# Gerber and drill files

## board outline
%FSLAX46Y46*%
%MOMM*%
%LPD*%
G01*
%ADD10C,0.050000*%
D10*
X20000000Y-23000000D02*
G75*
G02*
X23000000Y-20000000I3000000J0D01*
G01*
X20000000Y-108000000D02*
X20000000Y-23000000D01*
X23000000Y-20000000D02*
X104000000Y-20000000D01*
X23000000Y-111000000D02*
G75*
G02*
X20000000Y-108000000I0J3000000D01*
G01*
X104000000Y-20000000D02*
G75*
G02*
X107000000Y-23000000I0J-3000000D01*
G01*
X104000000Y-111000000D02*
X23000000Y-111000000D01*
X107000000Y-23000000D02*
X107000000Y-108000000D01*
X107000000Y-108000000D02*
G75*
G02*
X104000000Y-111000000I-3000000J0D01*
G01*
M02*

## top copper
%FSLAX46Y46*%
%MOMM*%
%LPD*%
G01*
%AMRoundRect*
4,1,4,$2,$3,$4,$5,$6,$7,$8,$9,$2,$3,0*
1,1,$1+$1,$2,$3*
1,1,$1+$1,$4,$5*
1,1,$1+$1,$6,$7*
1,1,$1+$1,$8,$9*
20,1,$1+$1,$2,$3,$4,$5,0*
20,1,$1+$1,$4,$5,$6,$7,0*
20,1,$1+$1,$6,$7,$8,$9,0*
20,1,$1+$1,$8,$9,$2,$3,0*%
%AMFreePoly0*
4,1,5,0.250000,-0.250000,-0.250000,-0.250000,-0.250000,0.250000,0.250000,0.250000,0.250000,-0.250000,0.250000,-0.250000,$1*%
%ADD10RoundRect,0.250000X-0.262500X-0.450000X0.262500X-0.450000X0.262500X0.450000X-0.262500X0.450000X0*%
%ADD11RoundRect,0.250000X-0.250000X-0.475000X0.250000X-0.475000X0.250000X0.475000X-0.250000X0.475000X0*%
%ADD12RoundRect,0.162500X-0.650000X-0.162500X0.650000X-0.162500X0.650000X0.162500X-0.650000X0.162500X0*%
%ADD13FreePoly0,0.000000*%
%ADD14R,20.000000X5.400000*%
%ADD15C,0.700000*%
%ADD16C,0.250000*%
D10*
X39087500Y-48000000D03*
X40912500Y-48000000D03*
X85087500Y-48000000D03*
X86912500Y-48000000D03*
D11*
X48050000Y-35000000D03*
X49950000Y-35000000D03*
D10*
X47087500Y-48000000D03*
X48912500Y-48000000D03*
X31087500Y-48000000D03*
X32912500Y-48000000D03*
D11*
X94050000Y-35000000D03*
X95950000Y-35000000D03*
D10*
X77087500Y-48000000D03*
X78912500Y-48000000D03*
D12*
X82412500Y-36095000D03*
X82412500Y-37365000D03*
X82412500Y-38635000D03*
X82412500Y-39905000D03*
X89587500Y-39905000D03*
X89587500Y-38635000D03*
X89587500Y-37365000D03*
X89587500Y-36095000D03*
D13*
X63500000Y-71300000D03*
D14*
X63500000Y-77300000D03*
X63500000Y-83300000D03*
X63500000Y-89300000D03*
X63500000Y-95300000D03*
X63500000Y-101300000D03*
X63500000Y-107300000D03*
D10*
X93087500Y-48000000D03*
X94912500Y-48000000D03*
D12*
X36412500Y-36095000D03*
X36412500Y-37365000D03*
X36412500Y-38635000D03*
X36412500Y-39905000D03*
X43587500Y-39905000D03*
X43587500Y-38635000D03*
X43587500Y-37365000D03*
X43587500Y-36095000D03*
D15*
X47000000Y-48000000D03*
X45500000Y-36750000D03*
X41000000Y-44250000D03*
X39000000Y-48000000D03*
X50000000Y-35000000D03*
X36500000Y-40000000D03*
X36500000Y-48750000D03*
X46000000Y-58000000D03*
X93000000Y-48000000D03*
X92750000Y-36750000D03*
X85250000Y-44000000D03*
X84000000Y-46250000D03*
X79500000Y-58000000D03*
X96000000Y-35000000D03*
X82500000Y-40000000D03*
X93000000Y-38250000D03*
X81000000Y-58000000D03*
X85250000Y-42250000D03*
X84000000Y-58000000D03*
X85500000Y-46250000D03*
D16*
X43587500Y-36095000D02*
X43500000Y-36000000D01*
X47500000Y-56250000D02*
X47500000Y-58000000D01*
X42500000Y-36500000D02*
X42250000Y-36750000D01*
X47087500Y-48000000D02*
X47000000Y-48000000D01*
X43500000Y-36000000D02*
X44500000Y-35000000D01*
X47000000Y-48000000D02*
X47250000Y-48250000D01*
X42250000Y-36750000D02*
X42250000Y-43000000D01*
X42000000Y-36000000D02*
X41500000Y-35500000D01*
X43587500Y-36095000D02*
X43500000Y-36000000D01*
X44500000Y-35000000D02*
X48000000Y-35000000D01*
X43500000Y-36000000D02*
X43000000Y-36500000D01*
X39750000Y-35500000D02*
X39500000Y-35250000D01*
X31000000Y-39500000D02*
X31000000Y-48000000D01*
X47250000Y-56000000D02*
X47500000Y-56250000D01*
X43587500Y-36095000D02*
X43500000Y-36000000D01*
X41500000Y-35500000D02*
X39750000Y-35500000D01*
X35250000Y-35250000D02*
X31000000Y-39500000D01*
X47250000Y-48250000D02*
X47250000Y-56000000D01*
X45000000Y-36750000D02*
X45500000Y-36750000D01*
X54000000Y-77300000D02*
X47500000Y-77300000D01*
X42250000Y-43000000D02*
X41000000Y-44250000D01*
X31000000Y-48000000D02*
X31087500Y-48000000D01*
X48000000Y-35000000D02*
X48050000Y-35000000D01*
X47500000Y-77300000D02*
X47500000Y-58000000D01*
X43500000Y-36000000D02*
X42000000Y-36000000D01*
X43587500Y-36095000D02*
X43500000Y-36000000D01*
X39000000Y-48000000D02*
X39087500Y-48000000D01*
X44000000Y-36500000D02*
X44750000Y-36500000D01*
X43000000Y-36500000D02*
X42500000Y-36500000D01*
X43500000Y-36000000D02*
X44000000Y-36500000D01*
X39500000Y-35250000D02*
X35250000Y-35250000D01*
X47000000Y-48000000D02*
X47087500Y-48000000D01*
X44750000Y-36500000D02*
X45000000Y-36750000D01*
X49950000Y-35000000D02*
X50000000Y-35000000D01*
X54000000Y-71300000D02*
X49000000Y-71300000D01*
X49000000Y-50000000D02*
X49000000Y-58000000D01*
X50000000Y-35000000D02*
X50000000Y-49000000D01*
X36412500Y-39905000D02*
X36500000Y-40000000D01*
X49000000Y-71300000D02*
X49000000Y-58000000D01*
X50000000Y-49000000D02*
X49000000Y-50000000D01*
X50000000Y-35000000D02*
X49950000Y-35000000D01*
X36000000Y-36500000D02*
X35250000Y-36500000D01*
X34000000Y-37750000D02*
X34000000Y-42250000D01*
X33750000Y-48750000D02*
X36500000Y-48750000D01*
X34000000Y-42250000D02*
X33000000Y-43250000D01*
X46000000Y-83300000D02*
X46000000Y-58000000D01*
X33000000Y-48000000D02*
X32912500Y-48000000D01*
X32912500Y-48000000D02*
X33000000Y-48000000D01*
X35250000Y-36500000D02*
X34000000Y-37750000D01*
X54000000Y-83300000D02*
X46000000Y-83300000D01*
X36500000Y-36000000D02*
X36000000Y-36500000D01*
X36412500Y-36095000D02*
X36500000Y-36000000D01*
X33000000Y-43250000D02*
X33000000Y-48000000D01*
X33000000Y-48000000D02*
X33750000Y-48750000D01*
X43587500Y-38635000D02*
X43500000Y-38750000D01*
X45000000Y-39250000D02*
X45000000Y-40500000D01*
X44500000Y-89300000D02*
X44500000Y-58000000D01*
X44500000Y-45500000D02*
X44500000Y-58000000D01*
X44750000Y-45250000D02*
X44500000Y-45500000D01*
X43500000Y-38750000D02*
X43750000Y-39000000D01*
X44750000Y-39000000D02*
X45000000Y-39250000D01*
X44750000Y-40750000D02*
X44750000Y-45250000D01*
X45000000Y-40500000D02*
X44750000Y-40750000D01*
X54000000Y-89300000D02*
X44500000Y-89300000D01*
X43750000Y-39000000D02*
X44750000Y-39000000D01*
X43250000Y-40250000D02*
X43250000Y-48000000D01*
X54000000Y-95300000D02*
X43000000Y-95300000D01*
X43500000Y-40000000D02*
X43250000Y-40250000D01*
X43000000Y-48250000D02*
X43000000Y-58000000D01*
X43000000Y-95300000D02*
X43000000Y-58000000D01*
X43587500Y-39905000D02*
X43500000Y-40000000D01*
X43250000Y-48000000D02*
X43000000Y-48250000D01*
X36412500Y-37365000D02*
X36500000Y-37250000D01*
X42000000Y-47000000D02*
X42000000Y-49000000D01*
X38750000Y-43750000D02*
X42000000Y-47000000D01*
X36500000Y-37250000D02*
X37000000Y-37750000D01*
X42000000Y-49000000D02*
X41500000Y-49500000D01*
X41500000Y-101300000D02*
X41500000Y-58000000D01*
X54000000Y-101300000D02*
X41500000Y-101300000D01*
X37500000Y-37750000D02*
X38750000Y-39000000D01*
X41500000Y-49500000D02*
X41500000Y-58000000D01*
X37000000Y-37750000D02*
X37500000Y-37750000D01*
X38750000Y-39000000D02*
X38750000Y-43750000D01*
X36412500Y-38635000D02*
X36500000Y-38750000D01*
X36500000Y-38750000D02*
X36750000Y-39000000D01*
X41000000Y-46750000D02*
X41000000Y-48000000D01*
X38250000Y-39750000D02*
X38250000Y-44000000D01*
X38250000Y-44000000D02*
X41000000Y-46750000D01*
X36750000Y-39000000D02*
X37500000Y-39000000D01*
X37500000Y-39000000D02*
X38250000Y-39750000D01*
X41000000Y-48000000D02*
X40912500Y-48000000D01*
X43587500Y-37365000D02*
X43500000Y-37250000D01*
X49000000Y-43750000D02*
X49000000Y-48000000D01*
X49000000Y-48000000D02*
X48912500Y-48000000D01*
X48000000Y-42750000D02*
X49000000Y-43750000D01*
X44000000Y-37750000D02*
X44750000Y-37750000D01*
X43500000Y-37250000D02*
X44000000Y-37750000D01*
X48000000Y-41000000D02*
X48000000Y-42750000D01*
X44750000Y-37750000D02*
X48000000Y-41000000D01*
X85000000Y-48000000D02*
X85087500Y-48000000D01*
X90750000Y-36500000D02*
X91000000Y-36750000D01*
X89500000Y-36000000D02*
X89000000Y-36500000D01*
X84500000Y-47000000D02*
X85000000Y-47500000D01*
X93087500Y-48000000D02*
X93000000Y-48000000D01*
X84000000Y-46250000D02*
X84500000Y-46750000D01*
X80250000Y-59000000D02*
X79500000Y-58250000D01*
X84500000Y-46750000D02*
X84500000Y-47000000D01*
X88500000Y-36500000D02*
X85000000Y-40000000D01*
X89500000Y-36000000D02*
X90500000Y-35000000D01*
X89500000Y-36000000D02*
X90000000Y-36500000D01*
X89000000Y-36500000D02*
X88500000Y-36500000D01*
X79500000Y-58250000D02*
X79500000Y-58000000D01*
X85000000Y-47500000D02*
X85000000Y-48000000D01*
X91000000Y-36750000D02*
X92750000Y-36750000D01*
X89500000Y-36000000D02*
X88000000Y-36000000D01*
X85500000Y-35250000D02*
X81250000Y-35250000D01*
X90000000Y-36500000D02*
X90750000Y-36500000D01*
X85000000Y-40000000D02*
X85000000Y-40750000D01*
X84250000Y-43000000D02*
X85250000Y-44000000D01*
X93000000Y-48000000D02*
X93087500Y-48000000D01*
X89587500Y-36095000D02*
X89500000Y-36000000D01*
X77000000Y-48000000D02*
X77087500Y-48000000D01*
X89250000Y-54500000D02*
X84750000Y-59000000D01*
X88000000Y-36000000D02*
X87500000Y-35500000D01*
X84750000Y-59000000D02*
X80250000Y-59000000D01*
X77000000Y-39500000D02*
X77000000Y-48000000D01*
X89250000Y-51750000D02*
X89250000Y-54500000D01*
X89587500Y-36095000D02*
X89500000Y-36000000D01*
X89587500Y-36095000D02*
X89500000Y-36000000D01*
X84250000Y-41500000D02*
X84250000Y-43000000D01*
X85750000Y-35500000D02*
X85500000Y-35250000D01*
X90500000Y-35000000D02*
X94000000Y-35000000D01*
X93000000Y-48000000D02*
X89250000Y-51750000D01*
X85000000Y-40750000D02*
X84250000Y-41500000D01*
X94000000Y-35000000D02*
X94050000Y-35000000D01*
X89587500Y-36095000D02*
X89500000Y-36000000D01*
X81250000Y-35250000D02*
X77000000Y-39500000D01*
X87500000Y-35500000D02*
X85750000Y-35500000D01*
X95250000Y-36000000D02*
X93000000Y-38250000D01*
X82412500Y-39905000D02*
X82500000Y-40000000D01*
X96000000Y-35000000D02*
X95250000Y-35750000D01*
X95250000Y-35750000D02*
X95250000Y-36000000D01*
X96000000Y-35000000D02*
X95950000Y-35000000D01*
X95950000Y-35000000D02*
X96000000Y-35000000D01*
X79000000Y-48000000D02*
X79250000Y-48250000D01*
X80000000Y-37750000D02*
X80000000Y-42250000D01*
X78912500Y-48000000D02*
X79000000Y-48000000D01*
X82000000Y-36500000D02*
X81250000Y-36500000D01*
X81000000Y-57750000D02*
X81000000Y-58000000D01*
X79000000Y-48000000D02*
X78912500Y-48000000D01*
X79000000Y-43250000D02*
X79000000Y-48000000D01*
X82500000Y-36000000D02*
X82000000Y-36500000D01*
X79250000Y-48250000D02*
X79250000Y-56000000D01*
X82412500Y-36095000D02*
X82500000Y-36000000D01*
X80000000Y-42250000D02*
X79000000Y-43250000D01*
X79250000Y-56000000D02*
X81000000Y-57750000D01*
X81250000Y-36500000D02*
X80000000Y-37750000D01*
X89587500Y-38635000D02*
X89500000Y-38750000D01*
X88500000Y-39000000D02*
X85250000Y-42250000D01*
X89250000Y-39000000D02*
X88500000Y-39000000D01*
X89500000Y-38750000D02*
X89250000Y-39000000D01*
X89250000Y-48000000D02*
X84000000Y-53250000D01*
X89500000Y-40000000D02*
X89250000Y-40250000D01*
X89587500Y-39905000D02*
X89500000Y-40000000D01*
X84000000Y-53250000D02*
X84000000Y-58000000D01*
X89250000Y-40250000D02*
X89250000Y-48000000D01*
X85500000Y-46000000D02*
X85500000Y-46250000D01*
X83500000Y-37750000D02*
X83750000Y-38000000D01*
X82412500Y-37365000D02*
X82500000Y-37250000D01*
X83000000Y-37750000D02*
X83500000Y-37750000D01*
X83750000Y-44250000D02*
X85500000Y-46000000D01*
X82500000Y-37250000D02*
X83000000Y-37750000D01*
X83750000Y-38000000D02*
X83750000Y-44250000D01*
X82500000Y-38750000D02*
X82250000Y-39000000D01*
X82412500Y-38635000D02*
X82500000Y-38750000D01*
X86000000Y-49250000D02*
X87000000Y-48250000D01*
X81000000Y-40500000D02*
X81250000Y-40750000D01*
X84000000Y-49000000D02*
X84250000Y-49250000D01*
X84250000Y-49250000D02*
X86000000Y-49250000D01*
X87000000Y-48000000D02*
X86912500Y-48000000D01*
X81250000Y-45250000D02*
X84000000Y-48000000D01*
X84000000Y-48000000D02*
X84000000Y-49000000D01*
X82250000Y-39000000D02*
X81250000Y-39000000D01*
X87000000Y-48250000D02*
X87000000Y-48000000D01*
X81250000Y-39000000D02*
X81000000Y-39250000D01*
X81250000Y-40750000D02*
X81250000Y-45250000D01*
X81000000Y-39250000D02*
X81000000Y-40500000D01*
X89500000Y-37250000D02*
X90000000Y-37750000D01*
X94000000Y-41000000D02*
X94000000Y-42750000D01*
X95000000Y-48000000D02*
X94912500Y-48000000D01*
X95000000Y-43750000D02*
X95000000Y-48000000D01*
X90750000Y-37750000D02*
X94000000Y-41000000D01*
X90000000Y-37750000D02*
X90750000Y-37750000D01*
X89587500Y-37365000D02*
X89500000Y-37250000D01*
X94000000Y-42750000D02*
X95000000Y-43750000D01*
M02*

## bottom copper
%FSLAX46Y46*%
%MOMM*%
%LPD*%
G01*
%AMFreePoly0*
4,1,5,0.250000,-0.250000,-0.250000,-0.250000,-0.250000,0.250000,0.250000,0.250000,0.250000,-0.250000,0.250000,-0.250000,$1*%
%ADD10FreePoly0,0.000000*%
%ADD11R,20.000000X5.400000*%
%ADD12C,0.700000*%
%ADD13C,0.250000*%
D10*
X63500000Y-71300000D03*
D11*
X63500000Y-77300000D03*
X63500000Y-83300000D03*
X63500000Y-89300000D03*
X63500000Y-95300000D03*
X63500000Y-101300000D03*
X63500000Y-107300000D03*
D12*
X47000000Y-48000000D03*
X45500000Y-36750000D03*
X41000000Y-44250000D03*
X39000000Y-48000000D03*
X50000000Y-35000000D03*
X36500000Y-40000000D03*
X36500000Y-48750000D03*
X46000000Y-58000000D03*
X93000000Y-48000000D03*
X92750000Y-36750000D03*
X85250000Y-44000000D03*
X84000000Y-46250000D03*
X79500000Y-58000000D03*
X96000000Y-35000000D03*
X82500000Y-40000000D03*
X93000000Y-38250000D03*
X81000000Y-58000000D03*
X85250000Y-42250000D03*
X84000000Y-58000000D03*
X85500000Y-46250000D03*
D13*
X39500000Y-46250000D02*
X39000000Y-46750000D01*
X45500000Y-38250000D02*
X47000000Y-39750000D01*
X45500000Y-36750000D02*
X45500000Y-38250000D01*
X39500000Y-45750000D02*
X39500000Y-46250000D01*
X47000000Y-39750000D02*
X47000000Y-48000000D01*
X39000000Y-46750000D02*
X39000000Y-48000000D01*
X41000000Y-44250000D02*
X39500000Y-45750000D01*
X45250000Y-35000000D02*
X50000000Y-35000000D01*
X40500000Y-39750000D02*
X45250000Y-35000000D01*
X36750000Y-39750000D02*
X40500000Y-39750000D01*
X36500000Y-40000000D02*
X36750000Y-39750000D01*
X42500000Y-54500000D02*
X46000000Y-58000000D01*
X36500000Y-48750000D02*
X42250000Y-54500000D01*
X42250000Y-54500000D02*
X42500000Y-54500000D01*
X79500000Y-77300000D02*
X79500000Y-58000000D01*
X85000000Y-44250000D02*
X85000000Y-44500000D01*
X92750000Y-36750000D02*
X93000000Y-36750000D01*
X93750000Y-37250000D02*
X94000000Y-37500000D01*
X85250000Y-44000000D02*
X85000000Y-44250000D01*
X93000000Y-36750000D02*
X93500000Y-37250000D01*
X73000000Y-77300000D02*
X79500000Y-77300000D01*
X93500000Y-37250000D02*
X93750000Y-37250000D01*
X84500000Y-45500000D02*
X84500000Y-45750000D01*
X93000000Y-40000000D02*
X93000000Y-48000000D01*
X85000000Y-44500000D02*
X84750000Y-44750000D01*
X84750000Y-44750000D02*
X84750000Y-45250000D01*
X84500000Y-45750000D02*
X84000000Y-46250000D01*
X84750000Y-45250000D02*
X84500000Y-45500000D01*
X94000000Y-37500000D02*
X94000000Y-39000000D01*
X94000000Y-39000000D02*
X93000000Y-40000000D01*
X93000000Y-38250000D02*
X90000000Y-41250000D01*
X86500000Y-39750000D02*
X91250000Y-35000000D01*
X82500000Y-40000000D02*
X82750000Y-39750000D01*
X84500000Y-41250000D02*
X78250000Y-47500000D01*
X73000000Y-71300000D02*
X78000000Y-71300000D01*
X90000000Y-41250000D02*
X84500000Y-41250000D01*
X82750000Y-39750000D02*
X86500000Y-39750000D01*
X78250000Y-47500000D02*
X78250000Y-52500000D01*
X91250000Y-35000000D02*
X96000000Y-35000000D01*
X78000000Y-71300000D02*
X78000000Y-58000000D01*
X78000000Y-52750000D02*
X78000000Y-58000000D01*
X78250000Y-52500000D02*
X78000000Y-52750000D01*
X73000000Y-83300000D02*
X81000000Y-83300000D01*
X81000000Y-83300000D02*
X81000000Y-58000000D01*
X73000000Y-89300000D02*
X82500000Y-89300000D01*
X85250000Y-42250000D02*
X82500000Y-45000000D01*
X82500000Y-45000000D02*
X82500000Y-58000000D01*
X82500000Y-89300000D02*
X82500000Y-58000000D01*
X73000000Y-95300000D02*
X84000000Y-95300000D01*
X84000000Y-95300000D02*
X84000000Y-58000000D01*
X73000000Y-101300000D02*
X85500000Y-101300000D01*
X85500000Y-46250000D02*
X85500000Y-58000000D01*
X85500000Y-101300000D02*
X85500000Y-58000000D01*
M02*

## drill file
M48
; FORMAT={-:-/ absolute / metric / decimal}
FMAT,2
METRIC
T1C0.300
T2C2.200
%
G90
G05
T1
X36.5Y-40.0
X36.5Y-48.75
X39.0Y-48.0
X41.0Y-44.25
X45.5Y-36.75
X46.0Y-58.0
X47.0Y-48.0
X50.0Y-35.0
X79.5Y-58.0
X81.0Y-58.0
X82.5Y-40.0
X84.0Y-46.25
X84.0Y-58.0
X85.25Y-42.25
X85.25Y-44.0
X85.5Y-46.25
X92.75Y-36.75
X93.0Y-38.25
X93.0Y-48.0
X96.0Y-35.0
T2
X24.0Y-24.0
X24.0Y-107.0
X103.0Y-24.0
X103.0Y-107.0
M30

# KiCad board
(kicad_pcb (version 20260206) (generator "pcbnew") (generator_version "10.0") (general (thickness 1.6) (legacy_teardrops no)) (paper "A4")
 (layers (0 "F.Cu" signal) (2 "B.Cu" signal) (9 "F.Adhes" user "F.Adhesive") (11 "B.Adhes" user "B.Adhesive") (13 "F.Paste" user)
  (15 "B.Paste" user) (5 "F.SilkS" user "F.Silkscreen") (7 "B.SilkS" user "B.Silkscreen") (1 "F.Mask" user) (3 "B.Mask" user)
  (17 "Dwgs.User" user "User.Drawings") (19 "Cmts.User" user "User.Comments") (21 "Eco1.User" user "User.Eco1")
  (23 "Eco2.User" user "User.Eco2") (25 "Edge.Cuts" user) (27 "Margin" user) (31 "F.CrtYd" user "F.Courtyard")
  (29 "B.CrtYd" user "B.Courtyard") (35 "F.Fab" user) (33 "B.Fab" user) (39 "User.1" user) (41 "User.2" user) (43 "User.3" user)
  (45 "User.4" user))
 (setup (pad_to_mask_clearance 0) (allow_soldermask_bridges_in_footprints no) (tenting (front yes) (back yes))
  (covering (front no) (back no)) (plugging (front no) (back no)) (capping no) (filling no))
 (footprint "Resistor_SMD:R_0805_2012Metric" (layer "F.Cu") (at 40 48)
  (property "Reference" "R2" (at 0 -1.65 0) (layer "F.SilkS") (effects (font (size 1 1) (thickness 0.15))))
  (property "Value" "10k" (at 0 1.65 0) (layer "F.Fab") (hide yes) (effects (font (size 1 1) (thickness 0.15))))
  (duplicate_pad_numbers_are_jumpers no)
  (pad "1" smd roundrect (at -0.9125 0) (size 1.025 1.4) (layers "F.Cu" "F.Mask" "F.Paste") (roundrect_rratio 0.243902) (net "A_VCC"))
  (pad "2" smd roundrect (at 0.9125 0) (size 1.025 1.4) (layers "F.Cu" "F.Mask" "F.Paste") (roundrect_rratio 0.243902) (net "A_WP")))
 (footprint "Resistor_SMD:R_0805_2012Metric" (layer "F.Cu") (at 86 48)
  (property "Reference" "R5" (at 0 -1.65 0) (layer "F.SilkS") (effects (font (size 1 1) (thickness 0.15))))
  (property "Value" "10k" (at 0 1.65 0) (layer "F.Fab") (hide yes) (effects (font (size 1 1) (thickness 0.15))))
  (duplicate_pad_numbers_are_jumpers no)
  (pad "1" smd roundrect (at -0.9125 0) (size 1.025 1.4) (layers "F.Cu" "F.Mask" "F.Paste") (roundrect_rratio 0.243902) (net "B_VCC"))
  (pad "2" smd roundrect (at 0.9125 0) (size 1.025 1.4) (layers "F.Cu" "F.Mask" "F.Paste") (roundrect_rratio 0.243902) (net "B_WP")))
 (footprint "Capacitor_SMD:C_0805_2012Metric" (layer "F.Cu") (at 49 35)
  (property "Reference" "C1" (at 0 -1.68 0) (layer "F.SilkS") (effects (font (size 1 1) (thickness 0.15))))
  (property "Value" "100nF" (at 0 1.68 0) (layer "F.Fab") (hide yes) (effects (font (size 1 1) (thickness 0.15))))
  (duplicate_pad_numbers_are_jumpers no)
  (pad "1" smd roundrect (at -0.95 0) (size 1 1.45) (layers "F.Cu" "F.Mask" "F.Paste") (roundrect_rratio 0.25) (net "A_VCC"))
  (pad "2" smd roundrect (at 0.95 0) (size 1 1.45) (layers "F.Cu" "F.Mask" "F.Paste") (roundrect_rratio 0.25) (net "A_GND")))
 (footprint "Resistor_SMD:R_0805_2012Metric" (layer "F.Cu") (at 48 48)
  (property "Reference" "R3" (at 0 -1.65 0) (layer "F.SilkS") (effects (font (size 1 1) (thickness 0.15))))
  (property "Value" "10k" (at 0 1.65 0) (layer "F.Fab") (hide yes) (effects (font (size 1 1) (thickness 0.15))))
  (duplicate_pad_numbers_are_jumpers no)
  (pad "1" smd roundrect (at -0.9125 0) (size 1.025 1.4) (layers "F.Cu" "F.Mask" "F.Paste") (roundrect_rratio 0.243902) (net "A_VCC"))
  (pad "2" smd roundrect (at 0.9125 0) (size 1.025 1.4) (layers "F.Cu" "F.Mask" "F.Paste") (roundrect_rratio 0.243902) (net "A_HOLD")))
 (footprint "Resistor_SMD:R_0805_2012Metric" (layer "F.Cu") (at 32 48)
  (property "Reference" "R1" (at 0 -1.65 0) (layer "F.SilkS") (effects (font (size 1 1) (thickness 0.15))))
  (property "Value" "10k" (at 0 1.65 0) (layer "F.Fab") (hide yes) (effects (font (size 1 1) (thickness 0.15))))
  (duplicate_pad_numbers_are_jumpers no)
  (pad "1" smd roundrect (at -0.9125 0) (size 1.025 1.4) (layers "F.Cu" "F.Mask" "F.Paste") (roundrect_rratio 0.243902) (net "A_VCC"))
  (pad "2" smd roundrect (at 0.9125 0) (size 1.025 1.4) (layers "F.Cu" "F.Mask" "F.Paste") (roundrect_rratio 0.243902) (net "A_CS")))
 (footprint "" (layer "F.Cu") (at 103 107)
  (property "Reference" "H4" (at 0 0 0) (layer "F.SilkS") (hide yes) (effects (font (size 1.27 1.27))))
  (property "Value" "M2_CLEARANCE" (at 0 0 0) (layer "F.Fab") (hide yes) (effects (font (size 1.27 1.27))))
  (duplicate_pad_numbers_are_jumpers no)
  (pad "" np_thru_hole circle (at 0 0) (size 2.2 2.2) (drill 2.2) (layers "*.Cu")))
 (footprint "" (layer "F.Cu") (at 24 24)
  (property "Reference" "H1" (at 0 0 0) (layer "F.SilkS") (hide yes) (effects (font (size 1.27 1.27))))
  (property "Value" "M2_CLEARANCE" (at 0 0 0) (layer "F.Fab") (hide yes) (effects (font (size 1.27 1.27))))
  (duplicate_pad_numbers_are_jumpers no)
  (pad "" np_thru_hole circle (at 0 0) (size 2.2 2.2) (drill 2.2) (layers "*.Cu")))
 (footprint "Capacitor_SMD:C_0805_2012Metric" (layer "F.Cu") (at 95 35)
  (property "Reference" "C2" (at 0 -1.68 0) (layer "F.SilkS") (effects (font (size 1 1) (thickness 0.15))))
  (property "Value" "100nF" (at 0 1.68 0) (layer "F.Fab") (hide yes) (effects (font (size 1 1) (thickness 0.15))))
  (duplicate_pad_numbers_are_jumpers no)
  (pad "1" smd roundrect (at -0.95 0) (size 1 1.45) (layers "F.Cu" "F.Mask" "F.Paste") (roundrect_rratio 0.25) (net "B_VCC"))
  (pad "2" smd roundrect (at 0.95 0) (size 1 1.45) (layers "F.Cu" "F.Mask" "F.Paste") (roundrect_rratio 0.25) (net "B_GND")))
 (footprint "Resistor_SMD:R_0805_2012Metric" (layer "F.Cu") (at 78 48)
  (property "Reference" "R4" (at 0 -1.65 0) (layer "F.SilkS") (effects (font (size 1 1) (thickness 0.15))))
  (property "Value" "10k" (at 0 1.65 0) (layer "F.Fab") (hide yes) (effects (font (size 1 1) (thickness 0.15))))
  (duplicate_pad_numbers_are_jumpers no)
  (pad "1" smd roundrect (at -0.9125 0) (size 1.025 1.4) (layers "F.Cu" "F.Mask" "F.Paste") (roundrect_rratio 0.243902) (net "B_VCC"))
  (pad "2" smd roundrect (at 0.9125 0) (size 1.025 1.4) (layers "F.Cu" "F.Mask" "F.Paste") (roundrect_rratio 0.243902) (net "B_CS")))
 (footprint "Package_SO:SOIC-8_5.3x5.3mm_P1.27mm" (layer "F.Cu") (at 86 38)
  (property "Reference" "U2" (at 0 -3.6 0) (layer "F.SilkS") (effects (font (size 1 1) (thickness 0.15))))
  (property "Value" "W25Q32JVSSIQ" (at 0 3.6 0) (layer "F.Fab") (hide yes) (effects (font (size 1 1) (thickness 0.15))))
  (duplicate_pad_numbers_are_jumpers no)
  (pad "1" smd roundrect (at -3.5875 -1.905) (size 1.625 0.65) (layers "F.Cu" "F.Mask" "F.Paste") (roundrect_rratio 0.25) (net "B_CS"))
  (pad "2" smd roundrect (at -3.5875 -0.635) (size 1.625 0.65) (layers "F.Cu" "F.Mask" "F.Paste") (roundrect_rratio 0.25) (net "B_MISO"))
  (pad "3" smd roundrect (at -3.5875 0.635) (size 1.625 0.65) (layers "F.Cu" "F.Mask" "F.Paste") (roundrect_rratio 0.25) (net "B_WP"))
  (pad "4" smd roundrect (at -3.5875 1.905) (size 1.625 0.65) (layers "F.Cu" "F.Mask" "F.Paste") (roundrect_rratio 0.25) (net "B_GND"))
  (pad "5" smd roundrect (at 3.5875 1.905) (size 1.625 0.65) (layers "F.Cu" "F.Mask" "F.Paste") (roundrect_rratio 0.25) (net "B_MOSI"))
  (pad "6" smd roundrect (at 3.5875 0.635) (size 1.625 0.65) (layers "F.Cu" "F.Mask" "F.Paste") (roundrect_rratio 0.25) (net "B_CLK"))
  (pad "7" smd roundrect (at 3.5875 -0.635) (size 1.625 0.65) (layers "F.Cu" "F.Mask" "F.Paste") (roundrect_rratio 0.25) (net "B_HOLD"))
  (pad "8" smd roundrect (at 3.5875 -1.905) (size 1.625 0.65) (layers "F.Cu" "F.Mask" "F.Paste") (roundrect_rratio 0.25) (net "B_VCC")))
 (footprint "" (layer "F.Cu") (at 103 24)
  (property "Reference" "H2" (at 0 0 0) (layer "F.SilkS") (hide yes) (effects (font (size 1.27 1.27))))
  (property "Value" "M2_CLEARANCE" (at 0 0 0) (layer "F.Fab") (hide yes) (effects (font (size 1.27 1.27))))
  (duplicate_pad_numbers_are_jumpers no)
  (pad "" np_thru_hole circle (at 0 0) (size 2.2 2.2) (drill 2.2) (layers "*.Cu")))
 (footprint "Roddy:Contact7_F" (layer "F.Cu") (at 63.5 0)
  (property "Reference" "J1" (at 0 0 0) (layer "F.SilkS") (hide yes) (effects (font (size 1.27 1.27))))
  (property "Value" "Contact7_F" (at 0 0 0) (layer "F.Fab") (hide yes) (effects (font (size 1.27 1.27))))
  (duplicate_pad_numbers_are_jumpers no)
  (pad "1" smd custom (at 0 71.3) (size 0.5 0.5) (layers "F.Cu" "F.Mask") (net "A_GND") (solder_mask_margin 0.05) (thermal_bridge_angle 45)
   (options (clearance outline) (anchor rect)) (primitives))
  (pad "2" smd rect (at 0 77.3) (size 20 5.4) (layers "F.Cu" "F.Mask") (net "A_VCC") (solder_mask_margin 0.05) (thermal_bridge_angle 45))
  (pad "3" smd rect (at 0 83.3) (size 20 5.4) (layers "F.Cu" "F.Mask") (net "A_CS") (solder_mask_margin 0.05) (thermal_bridge_angle 45))
  (pad "4" smd rect (at 0 89.3) (size 20 5.4) (layers "F.Cu" "F.Mask") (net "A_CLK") (solder_mask_margin 0.05) (thermal_bridge_angle 45))
  (pad "5" smd rect (at 0 95.3) (size 20 5.4) (layers "F.Cu" "F.Mask") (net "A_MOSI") (solder_mask_margin 0.05) (thermal_bridge_angle 45))
  (pad "6" smd rect (at 0 101.3) (size 20 5.4) (layers "F.Cu" "F.Mask") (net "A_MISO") (solder_mask_margin 0.05) (thermal_bridge_angle 45))
  (pad "7" smd rect (at 0 107.3) (size 20 5.4) (layers "F.Cu" "F.Mask") (solder_mask_margin 0.05) (thermal_bridge_angle 45)))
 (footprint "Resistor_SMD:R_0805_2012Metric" (layer "F.Cu") (at 94 48)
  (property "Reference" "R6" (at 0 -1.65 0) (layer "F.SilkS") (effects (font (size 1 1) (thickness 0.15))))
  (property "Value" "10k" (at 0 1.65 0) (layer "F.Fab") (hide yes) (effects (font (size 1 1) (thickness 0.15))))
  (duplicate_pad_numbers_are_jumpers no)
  (pad "1" smd roundrect (at -0.9125 0) (size 1.025 1.4) (layers "F.Cu" "F.Mask" "F.Paste") (roundrect_rratio 0.243902) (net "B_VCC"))
  (pad "2" smd roundrect (at 0.9125 0) (size 1.025 1.4) (layers "F.Cu" "F.Mask" "F.Paste") (roundrect_rratio 0.243902) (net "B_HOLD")))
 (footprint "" (layer "F.Cu") (at 24 107)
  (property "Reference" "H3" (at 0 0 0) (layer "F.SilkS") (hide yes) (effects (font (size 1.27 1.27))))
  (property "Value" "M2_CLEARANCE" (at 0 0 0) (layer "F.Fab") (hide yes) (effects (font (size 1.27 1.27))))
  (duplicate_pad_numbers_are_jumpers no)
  (pad "" np_thru_hole circle (at 0 0) (size 2.2 2.2) (drill 2.2) (layers "*.Cu")))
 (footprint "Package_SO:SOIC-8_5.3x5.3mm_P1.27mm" (layer "F.Cu") (at 40 38)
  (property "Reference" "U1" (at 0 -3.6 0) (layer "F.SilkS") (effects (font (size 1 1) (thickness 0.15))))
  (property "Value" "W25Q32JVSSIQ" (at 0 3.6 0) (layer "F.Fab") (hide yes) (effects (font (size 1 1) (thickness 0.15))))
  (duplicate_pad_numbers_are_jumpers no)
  (pad "1" smd roundrect (at -3.5875 -1.905) (size 1.625 0.65) (layers "F.Cu" "F.Mask" "F.Paste") (roundrect_rratio 0.25) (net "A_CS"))
  (pad "2" smd roundrect (at -3.5875 -0.635) (size 1.625 0.65) (layers "F.Cu" "F.Mask" "F.Paste") (roundrect_rratio 0.25) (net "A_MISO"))
  (pad "3" smd roundrect (at -3.5875 0.635) (size 1.625 0.65) (layers "F.Cu" "F.Mask" "F.Paste") (roundrect_rratio 0.25) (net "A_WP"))
  (pad "4" smd roundrect (at -3.5875 1.905) (size 1.625 0.65) (layers "F.Cu" "F.Mask" "F.Paste") (roundrect_rratio 0.25) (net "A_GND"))
  (pad "5" smd roundrect (at 3.5875 1.905) (size 1.625 0.65) (layers "F.Cu" "F.Mask" "F.Paste") (roundrect_rratio 0.25) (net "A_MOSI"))
  (pad "6" smd roundrect (at 3.5875 0.635) (size 1.625 0.65) (layers "F.Cu" "F.Mask" "F.Paste") (roundrect_rratio 0.25) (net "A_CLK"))
  (pad "7" smd roundrect (at 3.5875 -0.635) (size 1.625 0.65) (layers "F.Cu" "F.Mask" "F.Paste") (roundrect_rratio 0.25) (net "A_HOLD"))
  (pad "8" smd roundrect (at 3.5875 -1.905) (size 1.625 0.65) (layers "F.Cu" "F.Mask" "F.Paste") (roundrect_rratio 0.25) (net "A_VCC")))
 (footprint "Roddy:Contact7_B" (layer "B.Cu") (at 63.5 0)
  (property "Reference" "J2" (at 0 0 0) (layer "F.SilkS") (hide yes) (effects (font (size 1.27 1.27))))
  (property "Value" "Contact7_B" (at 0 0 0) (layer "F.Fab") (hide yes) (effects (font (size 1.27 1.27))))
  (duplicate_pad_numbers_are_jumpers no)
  (pad "1" smd custom (at 0 71.3) (size 0.5 0.5) (layers "B.Cu" "B.Mask") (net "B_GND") (solder_mask_margin 0.05) (thermal_bridge_angle 45)
   (options (clearance outline) (anchor rect)) (primitives))
  (pad "2" smd rect (at 0 77.3) (size 20 5.4) (layers "B.Cu" "B.Mask") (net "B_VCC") (solder_mask_margin 0.05) (thermal_bridge_angle 45))
  (pad "3" smd rect (at 0 83.3) (size 20 5.4) (layers "B.Cu" "B.Mask") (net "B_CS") (solder_mask_margin 0.05) (thermal_bridge_angle 45))
  (pad "4" smd rect (at 0 89.3) (size 20 5.4) (layers "B.Cu" "B.Mask") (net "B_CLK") (solder_mask_margin 0.05) (thermal_bridge_angle 45))
  (pad "5" smd rect (at 0 95.3) (size 20 5.4) (layers "B.Cu" "B.Mask") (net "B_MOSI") (solder_mask_margin 0.05) (thermal_bridge_angle 45))
  (pad "6" smd rect (at 0 101.3) (size 20 5.4) (layers "B.Cu" "B.Mask") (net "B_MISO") (solder_mask_margin 0.05) (thermal_bridge_angle 45))
  (pad "7" smd rect (at 0 107.3) (size 20 5.4) (layers "B.Cu" "B.Mask") (solder_mask_margin 0.05) (thermal_bridge_angle 45)))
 (gr_arc (start 20 23) (mid 20.878679 20.878679) (end 23 20) (stroke (width 0.05) (type default)) (layer "Edge.Cuts"))
 (gr_line (start 20 108) (end 20 23) (stroke (width 0.05) (type default)) (layer "Edge.Cuts"))
 (gr_line (start 23 20) (end 104 20) (stroke (width 0.05) (type default)) (layer "Edge.Cuts"))
 (gr_arc (start 23 111) (mid 20.878679 110.12132) (end 20 108) (stroke (width 0.05) (type default)) (layer "Edge.Cuts"))
 (gr_arc (start 104 20) (mid 106.12132 20.878679) (end 107 23) (stroke (width 0.05) (type default)) (layer "Edge.Cuts"))
 (gr_line (start 104 111) (end 23 111) (stroke (width 0.05) (type default)) (layer "Edge.Cuts"))
 (gr_line (start 107 23) (end 107 108) (stroke (width 0.05) (type default)) (layer "Edge.Cuts"))
 (gr_arc (start 107 108) (mid 106.12132 110.12132) (end 104 111) (stroke (width 0.05) (type default)) (layer "Edge.Cuts"))
 (segment (start 43.5875 36.095) (end 43.5 36) (width 0.25) (layer "F.Cu") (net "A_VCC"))
 (segment (start 47.5 56.25) (end 47.5 58) (width 0.25) (layer "F.Cu") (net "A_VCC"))
 (segment (start 42.5 36.5) (end 42.25 36.75) (width 0.25) (layer "F.Cu") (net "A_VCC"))
 (segment (start 47.0875 48) (end 47 48) (width 0.25) (layer "F.Cu") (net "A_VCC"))
 (segment (start 43.5 36) (end 44.5 35) (width 0.25) (layer "F.Cu") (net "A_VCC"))
 (segment (start 47 48) (end 47.25 48.25) (width 0.25) (layer "F.Cu") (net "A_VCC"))
 (segment (start 42.25 36.75) (end 42.25 43) (width 0.25) (layer "F.Cu") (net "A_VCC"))
 (segment (start 42 36) (end 41.5 35.5) (width 0.25) (layer "F.Cu") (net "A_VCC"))
 (segment (start 43.5875 36.095) (end 43.5 36) (width 0.25) (layer "F.Cu") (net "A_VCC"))
 (segment (start 44.5 35) (end 48 35) (width 0.25) (layer "F.Cu") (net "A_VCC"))
 (segment (start 43.5 36) (end 43 36.5) (width 0.25) (layer "F.Cu") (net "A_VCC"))
 (segment (start 39.75 35.5) (end 39.5 35.25) (width 0.25) (layer "F.Cu") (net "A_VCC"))
 (segment (start 31 39.5) (end 31 48) (width 0.25) (layer "F.Cu") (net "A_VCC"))
 (segment (start 47.25 56) (end 47.5 56.25) (width 0.25) (layer "F.Cu") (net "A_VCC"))
 (segment (start 43.5875 36.095) (end 43.5 36) (width 0.25) (layer "F.Cu") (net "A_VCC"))
 (segment (start 41.5 35.5) (end 39.75 35.5) (width 0.25) (layer "F.Cu") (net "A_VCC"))
 (segment (start 35.25 35.25) (end 31 39.5) (width 0.25) (layer "F.Cu") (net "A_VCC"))
 (segment (start 47.25 48.25) (end 47.25 56) (width 0.25) (layer "F.Cu") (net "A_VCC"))
 (segment (start 45 36.75) (end 45.5 36.75) (width 0.25) (layer "F.Cu") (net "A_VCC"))
 (segment (start 54 77.3) (end 47.5 77.3) (width 0.25) (layer "F.Cu") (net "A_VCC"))
 (segment (start 42.25 43) (end 41 44.25) (width 0.25) (layer "F.Cu") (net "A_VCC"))
 (segment (start 31 48) (end 31.0875 48) (width 0.25) (layer "F.Cu") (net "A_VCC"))
 (segment (start 48 35) (end 48.05 35) (width 0.25) (layer "F.Cu") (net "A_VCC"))
 (segment (start 47.5 77.3) (end 47.5 58) (width 0.25) (layer "F.Cu") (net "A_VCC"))
 (segment (start 43.5 36) (end 42 36) (width 0.25) (layer "F.Cu") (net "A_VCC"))
 (segment (start 43.5875 36.095) (end 43.5 36) (width 0.25) (layer "F.Cu") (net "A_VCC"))
 (segment (start 39 48) (end 39.0875 48) (width 0.25) (layer "F.Cu") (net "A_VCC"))
 (segment (start 44 36.5) (end 44.75 36.5) (width 0.25) (layer "F.Cu") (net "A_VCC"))
 (segment (start 43 36.5) (end 42.5 36.5) (width 0.25) (layer "F.Cu") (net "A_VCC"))
 (segment (start 43.5 36) (end 44 36.5) (width 0.25) (layer "F.Cu") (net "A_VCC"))
 (segment (start 39.5 35.25) (end 35.25 35.25) (width 0.25) (layer "F.Cu") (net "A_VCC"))
 (segment (start 47 48) (end 47.0875 48) (width 0.25) (layer "F.Cu") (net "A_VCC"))
 (segment (start 44.75 36.5) (end 45 36.75) (width 0.25) (layer "F.Cu") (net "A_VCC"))
 (via (at 47 48) (size 0.7) (drill 0.3) (layers "F.Cu" "B.Cu") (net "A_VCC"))
 (via (at 45.5 36.75) (size 0.7) (drill 0.3) (layers "F.Cu" "B.Cu") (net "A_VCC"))
 (via (at 41 44.25) (size 0.7) (drill 0.3) (layers "F.Cu" "B.Cu") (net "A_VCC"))
 (via (at 39 48) (size 0.7) (drill 0.3) (layers "F.Cu" "B.Cu") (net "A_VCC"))
 (segment (start 39.5 46.25) (end 39 46.75) (width 0.25) (layer "B.Cu") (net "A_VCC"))
 (segment (start 45.5 38.25) (end 47 39.75) (width 0.25) (layer "B.Cu") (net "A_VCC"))
 (segment (start 45.5 36.75) (end 45.5 38.25) (width 0.25) (layer "B.Cu") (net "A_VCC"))
 (segment (start 39.5 45.75) (end 39.5 46.25) (width 0.25) (layer "B.Cu") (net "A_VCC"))
 (segment (start 47 39.75) (end 47 48) (width 0.25) (layer "B.Cu") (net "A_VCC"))
 (segment (start 39 46.75) (end 39 48) (width 0.25) (layer "B.Cu") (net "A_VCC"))
 (segment (start 41 44.25) (end 39.5 45.75) (width 0.25) (layer "B.Cu") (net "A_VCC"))
 (segment (start 49.95 35) (end 50 35) (width 0.25) (layer "F.Cu") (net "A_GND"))
 (segment (start 54 71.3) (end 49 71.3) (width 0.25) (layer "F.Cu") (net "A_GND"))
 (segment (start 49 50) (end 49 58) (width 0.25) (layer "F.Cu") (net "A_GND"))
 (segment (start 50 35) (end 50 49) (width 0.25) (layer "F.Cu") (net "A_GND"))
 (segment (start 36.4125 39.905) (end 36.5 40) (width 0.25) (layer "F.Cu") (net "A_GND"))
 (segment (start 49 71.3) (end 49 58) (width 0.25) (layer "F.Cu") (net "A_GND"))
 (segment (start 50 49) (end 49 50) (width 0.25) (layer "F.Cu") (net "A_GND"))
 (segment (start 50 35) (end 49.95 35) (width 0.25) (layer "F.Cu") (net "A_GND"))
 (via (at 50 35) (size 0.7) (drill 0.3) (layers "F.Cu" "B.Cu") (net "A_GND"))
 (via (at 36.5 40) (size 0.7) (drill 0.3) (layers "F.Cu" "B.Cu") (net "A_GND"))
 (segment (start 45.25 35) (end 50 35) (width 0.25) (layer "B.Cu") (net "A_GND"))
 (segment (start 40.5 39.75) (end 45.25 35) (width 0.25) (layer "B.Cu") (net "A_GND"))
 (segment (start 36.75 39.75) (end 40.5 39.75) (width 0.25) (layer "B.Cu") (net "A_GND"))
 (segment (start 36.5 40) (end 36.75 39.75) (width 0.25) (layer "B.Cu") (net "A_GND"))
 (segment (start 36 36.5) (end 35.25 36.5) (width 0.25) (layer "F.Cu") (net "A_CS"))
 (segment (start 34 37.75) (end 34 42.25) (width 0.25) (layer "F.Cu") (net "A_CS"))
 (segment (start 33.75 48.75) (end 36.5 48.75) (width 0.25) (layer "F.Cu") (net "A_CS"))
 (segment (start 34 42.25) (end 33 43.25) (width 0.25) (layer "F.Cu") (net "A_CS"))
 (segment (start 46 83.3) (end 46 58) (width 0.25) (layer "F.Cu") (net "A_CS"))
 (segment (start 33 48) (end 32.9125 48) (width 0.25) (layer "F.Cu") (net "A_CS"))
 (segment (start 32.9125 48) (end 33 48) (width 0.25) (layer "F.Cu") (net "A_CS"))
 (segment (start 35.25 36.5) (end 34 37.75) (width 0.25) (layer "F.Cu") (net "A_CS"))
 (segment (start 54 83.3) (end 46 83.3) (width 0.25) (layer "F.Cu") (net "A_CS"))
 (segment (start 36.5 36) (end 36 36.5) (width 0.25) (layer "F.Cu") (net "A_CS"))
 (segment (start 36.4125 36.095) (end 36.5 36) (width 0.25) (layer "F.Cu") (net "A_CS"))
 (segment (start 33 43.25) (end 33 48) (width 0.25) (layer "F.Cu") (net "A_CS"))
 (segment (start 33 48) (end 33.75 48.75) (width 0.25) (layer "F.Cu") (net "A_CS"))
 (via (at 36.5 48.75) (size 0.7) (drill 0.3) (layers "F.Cu" "B.Cu") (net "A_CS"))
 (via (at 46 58) (size 0.7) (drill 0.3) (layers "F.Cu" "B.Cu") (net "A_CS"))
 (segment (start 42.5 54.5) (end 46 58) (width 0.25) (layer "B.Cu") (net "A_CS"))
 (segment (start 36.5 48.75) (end 42.25 54.5) (width 0.25) (layer "B.Cu") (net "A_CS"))
 (segment (start 42.25 54.5) (end 42.5 54.5) (width 0.25) (layer "B.Cu") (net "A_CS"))
 (segment (start 43.5875 38.635) (end 43.5 38.75) (width 0.25) (layer "F.Cu") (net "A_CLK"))
 (segment (start 45 39.25) (end 45 40.5) (width 0.25) (layer "F.Cu") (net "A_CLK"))
 (segment (start 44.5 89.3) (end 44.5 58) (width 0.25) (layer "F.Cu") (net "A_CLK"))
 (segment (start 44.5 45.5) (end 44.5 58) (width 0.25) (layer "F.Cu") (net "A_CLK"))
 (segment (start 44.75 45.25) (end 44.5 45.5) (width 0.25) (layer "F.Cu") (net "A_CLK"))
 (segment (start 43.5 38.75) (end 43.75 39) (width 0.25) (layer "F.Cu") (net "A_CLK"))
 (segment (start 44.75 39) (end 45 39.25) (width 0.25) (layer "F.Cu") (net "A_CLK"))
 (segment (start 44.75 40.75) (end 44.75 45.25) (width 0.25) (layer "F.Cu") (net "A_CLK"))
 (segment (start 45 40.5) (end 44.75 40.75) (width 0.25) (layer "F.Cu") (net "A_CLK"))
 (segment (start 54 89.3) (end 44.5 89.3) (width 0.25) (layer "F.Cu") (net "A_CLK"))
 (segment (start 43.75 39) (end 44.75 39) (width 0.25) (layer "F.Cu") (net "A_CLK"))
 (segment (start 43.25 40.25) (end 43.25 48) (width 0.25) (layer "F.Cu") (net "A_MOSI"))
 (segment (start 54 95.3) (end 43 95.3) (width 0.25) (layer "F.Cu") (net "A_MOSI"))
 (segment (start 43.5 40) (end 43.25 40.25) (width 0.25) (layer "F.Cu") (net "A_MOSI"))
 (segment (start 43 48.25) (end 43 58) (width 0.25) (layer "F.Cu") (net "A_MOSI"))
 (segment (start 43 95.3) (end 43 58) (width 0.25) (layer "F.Cu") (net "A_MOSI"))
 (segment (start 43.5875 39.905) (end 43.5 40) (width 0.25) (layer "F.Cu") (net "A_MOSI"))
 (segment (start 43.25 48) (end 43 48.25) (width 0.25) (layer "F.Cu") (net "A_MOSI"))
 (segment (start 36.4125 37.365) (end 36.5 37.25) (width 0.25) (layer "F.Cu") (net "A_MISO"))
 (segment (start 42 47) (end 42 49) (width 0.25) (layer "F.Cu") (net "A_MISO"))
 (segment (start 38.75 43.75) (end 42 47) (width 0.25) (layer "F.Cu") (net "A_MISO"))
 (segment (start 36.5 37.25) (end 37 37.75) (width 0.25) (layer "F.Cu") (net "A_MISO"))
 (segment (start 42 49) (end 41.5 49.5) (width 0.25) (layer "F.Cu") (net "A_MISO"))
 (segment (start 41.5 101.3) (end 41.5 58) (width 0.25) (layer "F.Cu") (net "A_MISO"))
 (segment (start 54 101.3) (end 41.5 101.3) (width 0.25) (layer "F.Cu") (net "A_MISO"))
 (segment (start 37.5 37.75) (end 38.75 39) (width 0.25) (layer "F.Cu") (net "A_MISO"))
 (segment (start 41.5 49.5) (end 41.5 58) (width 0.25) (layer "F.Cu") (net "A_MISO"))
 (segment (start 37 37.75) (end 37.5 37.75) (width 0.25) (layer "F.Cu") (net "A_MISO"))
 (segment (start 38.75 39) (end 38.75 43.75) (width 0.25) (layer "F.Cu") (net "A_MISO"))
 (segment (start 36.4125 38.635) (end 36.5 38.75) (width 0.25) (layer "F.Cu") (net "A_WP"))
 (segment (start 36.5 38.75) (end 36.75 39) (width 0.25) (layer "F.Cu") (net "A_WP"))
 (segment (start 41 46.75) (end 41 48) (width 0.25) (layer "F.Cu") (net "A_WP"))
 (segment (start 38.25 39.75) (end 38.25 44) (width 0.25) (layer "F.Cu") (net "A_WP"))
 (segment (start 38.25 44) (end 41 46.75) (width 0.25) (layer "F.Cu") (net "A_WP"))
 (segment (start 36.75 39) (end 37.5 39) (width 0.25) (layer "F.Cu") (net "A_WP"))
 (segment (start 37.5 39) (end 38.25 39.75) (width 0.25) (layer "F.Cu") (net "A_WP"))
 (segment (start 41 48) (end 40.9125 48) (width 0.25) (layer "F.Cu") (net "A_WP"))
 (segment (start 43.5875 37.365) (end 43.5 37.25) (width 0.25) (layer "F.Cu") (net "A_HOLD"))
 (segment (start 49 43.75) (end 49 48) (width 0.25) (layer "F.Cu") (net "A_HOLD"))
 (segment (start 49 48) (end 48.9125 48) (width 0.25) (layer "F.Cu") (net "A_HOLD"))
 (segment (start 48 42.75) (end 49 43.75) (width 0.25) (layer "F.Cu") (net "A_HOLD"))
 (segment (start 44 37.75) (end 44.75 37.75) (width 0.25) (layer "F.Cu") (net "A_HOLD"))
 (segment (start 43.5 37.25) (end 44 37.75) (width 0.25) (layer "F.Cu") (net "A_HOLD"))
 (segment (start 48 41) (end 48 42.75) (width 0.25) (layer "F.Cu") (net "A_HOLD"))
 (segment (start 44.75 37.75) (end 48 41) (width 0.25) (layer "F.Cu") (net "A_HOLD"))
 (segment (start 85 48) (end 85.0875 48) (width 0.25) (layer "F.Cu") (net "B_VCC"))
 (segment (start 90.75 36.5) (end 91 36.75) (width 0.25) (layer "F.Cu") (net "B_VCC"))
 (segment (start 89.5 36) (end 89 36.5) (width 0.25) (layer "F.Cu") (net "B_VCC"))
 (segment (start 84.5 47) (end 85 47.5) (width 0.25) (layer "F.Cu") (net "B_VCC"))
 (segment (start 93.0875 48) (end 93 48) (width 0.25) (layer "F.Cu") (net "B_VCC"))
 (segment (start 84 46.25) (end 84.5 46.75) (width 0.25) (layer "F.Cu") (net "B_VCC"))
 (segment (start 80.25 59) (end 79.5 58.25) (width 0.25) (layer "F.Cu") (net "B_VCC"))
 (segment (start 84.5 46.75) (end 84.5 47) (width 0.25) (layer "F.Cu") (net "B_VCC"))
 (segment (start 88.5 36.5) (end 85 40) (width 0.25) (layer "F.Cu") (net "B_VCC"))
 (segment (start 89.5 36) (end 90.5 35) (width 0.25) (layer "F.Cu") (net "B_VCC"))
 (segment (start 89.5 36) (end 90 36.5) (width 0.25) (layer "F.Cu") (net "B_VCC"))
 (segment (start 89 36.5) (end 88.5 36.5) (width 0.25) (layer "F.Cu") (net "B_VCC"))
 (segment (start 79.5 58.25) (end 79.5 58) (width 0.25) (layer "F.Cu") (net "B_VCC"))
 (segment (start 85 47.5) (end 85 48) (width 0.25) (layer "F.Cu") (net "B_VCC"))
 (segment (start 91 36.75) (end 92.75 36.75) (width 0.25) (layer "F.Cu") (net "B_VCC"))
 (segment (start 89.5 36) (end 88 36) (width 0.25) (layer "F.Cu") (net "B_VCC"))
 (segment (start 85.5 35.25) (end 81.25 35.25) (width 0.25) (layer "F.Cu") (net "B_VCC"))
 (segment (start 90 36.5) (end 90.75 36.5) (width 0.25) (layer "F.Cu") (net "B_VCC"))
 (segment (start 85 40) (end 85 40.75) (width 0.25) (layer "F.Cu") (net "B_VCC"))
 (segment (start 84.25 43) (end 85.25 44) (width 0.25) (layer "F.Cu") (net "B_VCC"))
 (segment (start 93 48) (end 93.0875 48) (width 0.25) (layer "F.Cu") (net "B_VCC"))
 (segment (start 89.5875 36.095) (end 89.5 36) (width 0.25) (layer "F.Cu") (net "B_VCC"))
 (segment (start 77 48) (end 77.0875 48) (width 0.25) (layer "F.Cu") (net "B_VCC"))
 (segment (start 89.25 54.5) (end 84.75 59) (width 0.25) (layer "F.Cu") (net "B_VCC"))
 (segment (start 88 36) (end 87.5 35.5) (width 0.25) (layer "F.Cu") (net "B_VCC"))
 (segment (start 84.75 59) (end 80.25 59) (width 0.25) (layer "F.Cu") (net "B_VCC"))
 (segment (start 77 39.5) (end 77 48) (width 0.25) (layer "F.Cu") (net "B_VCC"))
 (segment (start 89.25 51.75) (end 89.25 54.5) (width 0.25) (layer "F.Cu") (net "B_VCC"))
 (segment (start 89.5875 36.095) (end 89.5 36) (width 0.25) (layer "F.Cu") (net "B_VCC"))
 (segment (start 89.5875 36.095) (end 89.5 36) (width 0.25) (layer "F.Cu") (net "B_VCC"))
 (segment (start 84.25 41.5) (end 84.25 43) (width 0.25) (layer "F.Cu") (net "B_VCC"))
 (segment (start 85.75 35.5) (end 85.5 35.25) (width 0.25) (layer "F.Cu") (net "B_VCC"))
 (segment (start 90.5 35) (end 94 35) (width 0.25) (layer "F.Cu") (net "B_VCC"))
 (segment (start 93 48) (end 89.25 51.75) (width 0.25) (layer "F.Cu") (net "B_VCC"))
 (segment (start 85 40.75) (end 84.25 41.5) (width 0.25) (layer "F.Cu") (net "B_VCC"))
 (segment (start 94 35) (end 94.05 35) (width 0.25) (layer "F.Cu") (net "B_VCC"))
 (segment (start 89.5875 36.095) (end 89.5 36) (width 0.25) (layer "F.Cu") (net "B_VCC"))
 (segment (start 81.25 35.25) (end 77 39.5) (width 0.25) (layer "F.Cu") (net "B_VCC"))
 (segment (start 87.5 35.5) (end 85.75 35.5) (width 0.25) (layer "F.Cu") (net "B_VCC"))
 (via (at 93 48) (size 0.7) (drill 0.3) (layers "F.Cu" "B.Cu") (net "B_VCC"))
 (via (at 92.75 36.75) (size 0.7) (drill 0.3) (layers "F.Cu" "B.Cu") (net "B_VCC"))
 (via (at 85.25 44) (size 0.7) (drill 0.3) (layers "F.Cu" "B.Cu") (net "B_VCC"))
 (via (at 84 46.25) (size 0.7) (drill 0.3) (layers "F.Cu" "B.Cu") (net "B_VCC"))
 (via (at 79.5 58) (size 0.7) (drill 0.3) (layers "F.Cu" "B.Cu") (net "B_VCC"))
 (segment (start 79.5 77.3) (end 79.5 58) (width 0.25) (layer "B.Cu") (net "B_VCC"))
 (segment (start 85 44.25) (end 85 44.5) (width 0.25) (layer "B.Cu") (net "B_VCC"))
 (segment (start 92.75 36.75) (end 93 36.75) (width 0.25) (layer "B.Cu") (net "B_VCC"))
 (segment (start 93.75 37.25) (end 94 37.5) (width 0.25) (layer "B.Cu") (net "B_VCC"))
 (segment (start 85.25 44) (end 85 44.25) (width 0.25) (layer "B.Cu") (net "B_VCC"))
 (segment (start 93 36.75) (end 93.5 37.25) (width 0.25) (layer "B.Cu") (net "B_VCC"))
 (segment (start 73 77.3) (end 79.5 77.3) (width 0.25) (layer "B.Cu") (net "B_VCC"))
 (segment (start 93.5 37.25) (end 93.75 37.25) (width 0.25) (layer "B.Cu") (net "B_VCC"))
 (segment (start 84.5 45.5) (end 84.5 45.75) (width 0.25) (layer "B.Cu") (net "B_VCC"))
 (segment (start 93 40) (end 93 48) (width 0.25) (layer "B.Cu") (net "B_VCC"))
 (segment (start 85 44.5) (end 84.75 44.75) (width 0.25) (layer "B.Cu") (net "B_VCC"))
 (segment (start 84.75 44.75) (end 84.75 45.25) (width 0.25) (layer "B.Cu") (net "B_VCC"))
 (segment (start 84.5 45.75) (end 84 46.25) (width 0.25) (layer "B.Cu") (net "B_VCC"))
 (segment (start 84.75 45.25) (end 84.5 45.5) (width 0.25) (layer "B.Cu") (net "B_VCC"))
 (segment (start 94 37.5) (end 94 39) (width 0.25) (layer "B.Cu") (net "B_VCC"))
 (segment (start 94 39) (end 93 40) (width 0.25) (layer "B.Cu") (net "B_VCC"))
 (segment (start 95.25 36) (end 93 38.25) (width 0.25) (layer "F.Cu") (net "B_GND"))
 (segment (start 82.4125 39.905) (end 82.5 40) (width 0.25) (layer "F.Cu") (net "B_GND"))
 (segment (start 96 35) (end 95.25 35.75) (width 0.25) (layer "F.Cu") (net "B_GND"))
 (segment (start 95.25 35.75) (end 95.25 36) (width 0.25) (layer "F.Cu") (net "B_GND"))
 (segment (start 96 35) (end 95.95 35) (width 0.25) (layer "F.Cu") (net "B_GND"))
 (segment (start 95.95 35) (end 96 35) (width 0.25) (layer "F.Cu") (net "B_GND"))
 (via (at 96 35) (size 0.7) (drill 0.3) (layers "F.Cu" "B.Cu") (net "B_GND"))
 (via (at 82.5 40) (size 0.7) (drill 0.3) (layers "F.Cu" "B.Cu") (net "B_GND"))
 (via (at 93 38.25) (size 0.7) (drill 0.3) (layers "F.Cu" "B.Cu") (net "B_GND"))
 (segment (start 93 38.25) (end 90 41.25) (width 0.25) (layer "B.Cu") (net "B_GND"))
 (segment (start 86.5 39.75) (end 91.25 35) (width 0.25) (layer "B.Cu") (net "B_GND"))
 (segment (start 82.5 40) (end 82.75 39.75) (width 0.25) (layer "B.Cu") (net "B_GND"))
 (segment (start 84.5 41.25) (end 78.25 47.5) (width 0.25) (layer "B.Cu") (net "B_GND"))
 (segment (start 73 71.3) (end 78 71.3) (width 0.25) (layer "B.Cu") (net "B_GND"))
 (segment (start 90 41.25) (end 84.5 41.25) (width 0.25) (layer "B.Cu") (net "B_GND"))
 (segment (start 82.75 39.75) (end 86.5 39.75) (width 0.25) (layer "B.Cu") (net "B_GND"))
 (segment (start 78.25 47.5) (end 78.25 52.5) (width 0.25) (layer "B.Cu") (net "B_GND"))
 (segment (start 91.25 35) (end 96 35) (width 0.25) (layer "B.Cu") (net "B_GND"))
 (segment (start 78 71.3) (end 78 58) (width 0.25) (layer "B.Cu") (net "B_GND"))
 (segment (start 78 52.75) (end 78 58) (width 0.25) (layer "B.Cu") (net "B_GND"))
 (segment (start 78.25 52.5) (end 78 52.75) (width 0.25) (layer "B.Cu") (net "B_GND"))
 (segment (start 79 48) (end 79.25 48.25) (width 0.25) (layer "F.Cu") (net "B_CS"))
 (segment (start 80 37.75) (end 80 42.25) (width 0.25) (layer "F.Cu") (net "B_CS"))
 (segment (start 78.9125 48) (end 79 48) (width 0.25) (layer "F.Cu") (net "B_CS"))
 (segment (start 82 36.5) (end 81.25 36.5) (width 0.25) (layer "F.Cu") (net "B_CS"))
 (segment (start 81 57.75) (end 81 58) (width 0.25) (layer "F.Cu") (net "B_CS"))
 (segment (start 79 48) (end 78.9125 48) (width 0.25) (layer "F.Cu") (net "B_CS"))
 (segment (start 79 43.25) (end 79 48) (width 0.25) (layer "F.Cu") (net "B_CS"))
 (segment (start 82.5 36) (end 82 36.5) (width 0.25) (layer "F.Cu") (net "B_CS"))
 (segment (start 79.25 48.25) (end 79.25 56) (width 0.25) (layer "F.Cu") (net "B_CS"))
 (segment (start 82.4125 36.095) (end 82.5 36) (width 0.25) (layer "F.Cu") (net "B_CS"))
 (segment (start 80 42.25) (end 79 43.25) (width 0.25) (layer "F.Cu") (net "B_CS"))
 (segment (start 79.25 56) (end 81 57.75) (width 0.25) (layer "F.Cu") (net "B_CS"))
 (segment (start 81.25 36.5) (end 80 37.75) (width 0.25) (layer "F.Cu") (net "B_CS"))
 (via (at 81 58) (size 0.7) (drill 0.3) (layers "F.Cu" "B.Cu") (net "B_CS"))
 (segment (start 73 83.3) (end 81 83.3) (width 0.25) (layer "B.Cu") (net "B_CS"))
 (segment (start 81 83.3) (end 81 58) (width 0.25) (layer "B.Cu") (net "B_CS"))
 (segment (start 89.5875 38.635) (end 89.5 38.75) (width 0.25) (layer "F.Cu") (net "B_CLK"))
 (segment (start 88.5 39) (end 85.25 42.25) (width 0.25) (layer "F.Cu") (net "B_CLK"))
 (segment (start 89.25 39) (end 88.5 39) (width 0.25) (layer "F.Cu") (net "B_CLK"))
 (segment (start 89.5 38.75) (end 89.25 39) (width 0.25) (layer "F.Cu") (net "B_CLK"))
 (via (at 85.25 42.25) (size 0.7) (drill 0.3) (layers "F.Cu" "B.Cu") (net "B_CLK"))
 (segment (start 73 89.3) (end 82.5 89.3) (width 0.25) (layer "B.Cu") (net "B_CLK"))
 (segment (start 85.25 42.25) (end 82.5 45) (width 0.25) (layer "B.Cu") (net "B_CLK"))
 (segment (start 82.5 45) (end 82.5 58) (width 0.25) (layer "B.Cu") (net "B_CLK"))
 (segment (start 82.5 89.3) (end 82.5 58) (width 0.25) (layer "B.Cu") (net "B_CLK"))
 (segment (start 89.25 48) (end 84 53.25) (width 0.25) (layer "F.Cu") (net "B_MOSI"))
 (segment (start 89.5 40) (end 89.25 40.25) (width 0.25) (layer "F.Cu") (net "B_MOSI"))
 (segment (start 89.5875 39.905) (end 89.5 40) (width 0.25) (layer "F.Cu") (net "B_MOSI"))
 (segment (start 84 53.25) (end 84 58) (width 0.25) (layer "F.Cu") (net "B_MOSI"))
 (segment (start 89.25 40.25) (end 89.25 48) (width 0.25) (layer "F.Cu") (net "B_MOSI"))
 (via (at 84 58) (size 0.7) (drill 0.3) (layers "F.Cu" "B.Cu") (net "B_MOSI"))
 (segment (start 73 95.3) (end 84 95.3) (width 0.25) (layer "B.Cu") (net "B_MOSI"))
 (segment (start 84 95.3) (end 84 58) (width 0.25) (layer "B.Cu") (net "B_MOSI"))
 (segment (start 85.5 46) (end 85.5 46.25) (width 0.25) (layer "F.Cu") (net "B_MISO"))
 (segment (start 83.5 37.75) (end 83.75 38) (width 0.25) (layer "F.Cu") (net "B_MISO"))
 (segment (start 82.4125 37.365) (end 82.5 37.25) (width 0.25) (layer "F.Cu") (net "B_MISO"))
 (segment (start 83 37.75) (end 83.5 37.75) (width 0.25) (layer "F.Cu") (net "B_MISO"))
 (segment (start 83.75 44.25) (end 85.5 46) (width 0.25) (layer "F.Cu") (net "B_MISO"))
 (segment (start 82.5 37.25) (end 83 37.75) (width 0.25) (layer "F.Cu") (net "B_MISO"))
 (segment (start 83.75 38) (end 83.75 44.25) (width 0.25) (layer "F.Cu") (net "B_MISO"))
 (via (at 85.5 46.25) (size 0.7) (drill 0.3) (layers "F.Cu" "B.Cu") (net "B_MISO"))
 (segment (start 73 101.3) (end 85.5 101.3) (width 0.25) (layer "B.Cu") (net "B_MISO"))
 (segment (start 85.5 46.25) (end 85.5 58) (width 0.25) (layer "B.Cu") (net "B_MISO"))
 (segment (start 85.5 101.3) (end 85.5 58) (width 0.25) (layer "B.Cu") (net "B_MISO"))
 (segment (start 82.5 38.75) (end 82.25 39) (width 0.25) (layer "F.Cu") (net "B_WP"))
 (segment (start 82.4125 38.635) (end 82.5 38.75) (width 0.25) (layer "F.Cu") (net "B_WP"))
 (segment (start 86 49.25) (end 87 48.25) (width 0.25) (layer "F.Cu") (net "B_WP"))
 (segment (start 81 40.5) (end 81.25 40.75) (width 0.25) (layer "F.Cu") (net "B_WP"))
 (segment (start 84 49) (end 84.25 49.25) (width 0.25) (layer "F.Cu") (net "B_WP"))
 (segment (start 84.25 49.25) (end 86 49.25) (width 0.25) (layer "F.Cu") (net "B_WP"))
 (segment (start 87 48) (end 86.9125 48) (width 0.25) (layer "F.Cu") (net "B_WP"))
 (segment (start 81.25 45.25) (end 84 48) (width 0.25) (layer "F.Cu") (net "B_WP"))
 (segment (start 84 48) (end 84 49) (width 0.25) (layer "F.Cu") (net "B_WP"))
 (segment (start 82.25 39) (end 81.25 39) (width 0.25) (layer "F.Cu") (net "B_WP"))
 (segment (start 87 48.25) (end 87 48) (width 0.25) (layer "F.Cu") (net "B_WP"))
 (segment (start 81.25 39) (end 81 39.25) (width 0.25) (layer "F.Cu") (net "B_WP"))
 (segment (start 81.25 40.75) (end 81.25 45.25) (width 0.25) (layer "F.Cu") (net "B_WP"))
 (segment (start 81 39.25) (end 81 40.5) (width 0.25) (layer "F.Cu") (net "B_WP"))
 (segment (start 89.5 37.25) (end 90 37.75) (width 0.25) (layer "F.Cu") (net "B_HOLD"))
 (segment (start 94 41) (end 94 42.75) (width 0.25) (layer "F.Cu") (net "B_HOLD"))
 (segment (start 95 48) (end 94.9125 48) (width 0.25) (layer "F.Cu") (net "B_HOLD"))
 (segment (start 95 43.75) (end 95 48) (width 0.25) (layer "F.Cu") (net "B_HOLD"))
 (segment (start 90.75 37.75) (end 94 41) (width 0.25) (layer "F.Cu") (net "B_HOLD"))
 (segment (start 90 37.75) (end 90.75 37.75) (width 0.25) (layer "F.Cu") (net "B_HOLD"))
 (segment (start 89.5875 37.365) (end 89.5 37.25) (width 0.25) (layer "F.Cu") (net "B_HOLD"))
 (segment (start 94 42.75) (end 95 43.75) (width 0.25) (layer "F.Cu") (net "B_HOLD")))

